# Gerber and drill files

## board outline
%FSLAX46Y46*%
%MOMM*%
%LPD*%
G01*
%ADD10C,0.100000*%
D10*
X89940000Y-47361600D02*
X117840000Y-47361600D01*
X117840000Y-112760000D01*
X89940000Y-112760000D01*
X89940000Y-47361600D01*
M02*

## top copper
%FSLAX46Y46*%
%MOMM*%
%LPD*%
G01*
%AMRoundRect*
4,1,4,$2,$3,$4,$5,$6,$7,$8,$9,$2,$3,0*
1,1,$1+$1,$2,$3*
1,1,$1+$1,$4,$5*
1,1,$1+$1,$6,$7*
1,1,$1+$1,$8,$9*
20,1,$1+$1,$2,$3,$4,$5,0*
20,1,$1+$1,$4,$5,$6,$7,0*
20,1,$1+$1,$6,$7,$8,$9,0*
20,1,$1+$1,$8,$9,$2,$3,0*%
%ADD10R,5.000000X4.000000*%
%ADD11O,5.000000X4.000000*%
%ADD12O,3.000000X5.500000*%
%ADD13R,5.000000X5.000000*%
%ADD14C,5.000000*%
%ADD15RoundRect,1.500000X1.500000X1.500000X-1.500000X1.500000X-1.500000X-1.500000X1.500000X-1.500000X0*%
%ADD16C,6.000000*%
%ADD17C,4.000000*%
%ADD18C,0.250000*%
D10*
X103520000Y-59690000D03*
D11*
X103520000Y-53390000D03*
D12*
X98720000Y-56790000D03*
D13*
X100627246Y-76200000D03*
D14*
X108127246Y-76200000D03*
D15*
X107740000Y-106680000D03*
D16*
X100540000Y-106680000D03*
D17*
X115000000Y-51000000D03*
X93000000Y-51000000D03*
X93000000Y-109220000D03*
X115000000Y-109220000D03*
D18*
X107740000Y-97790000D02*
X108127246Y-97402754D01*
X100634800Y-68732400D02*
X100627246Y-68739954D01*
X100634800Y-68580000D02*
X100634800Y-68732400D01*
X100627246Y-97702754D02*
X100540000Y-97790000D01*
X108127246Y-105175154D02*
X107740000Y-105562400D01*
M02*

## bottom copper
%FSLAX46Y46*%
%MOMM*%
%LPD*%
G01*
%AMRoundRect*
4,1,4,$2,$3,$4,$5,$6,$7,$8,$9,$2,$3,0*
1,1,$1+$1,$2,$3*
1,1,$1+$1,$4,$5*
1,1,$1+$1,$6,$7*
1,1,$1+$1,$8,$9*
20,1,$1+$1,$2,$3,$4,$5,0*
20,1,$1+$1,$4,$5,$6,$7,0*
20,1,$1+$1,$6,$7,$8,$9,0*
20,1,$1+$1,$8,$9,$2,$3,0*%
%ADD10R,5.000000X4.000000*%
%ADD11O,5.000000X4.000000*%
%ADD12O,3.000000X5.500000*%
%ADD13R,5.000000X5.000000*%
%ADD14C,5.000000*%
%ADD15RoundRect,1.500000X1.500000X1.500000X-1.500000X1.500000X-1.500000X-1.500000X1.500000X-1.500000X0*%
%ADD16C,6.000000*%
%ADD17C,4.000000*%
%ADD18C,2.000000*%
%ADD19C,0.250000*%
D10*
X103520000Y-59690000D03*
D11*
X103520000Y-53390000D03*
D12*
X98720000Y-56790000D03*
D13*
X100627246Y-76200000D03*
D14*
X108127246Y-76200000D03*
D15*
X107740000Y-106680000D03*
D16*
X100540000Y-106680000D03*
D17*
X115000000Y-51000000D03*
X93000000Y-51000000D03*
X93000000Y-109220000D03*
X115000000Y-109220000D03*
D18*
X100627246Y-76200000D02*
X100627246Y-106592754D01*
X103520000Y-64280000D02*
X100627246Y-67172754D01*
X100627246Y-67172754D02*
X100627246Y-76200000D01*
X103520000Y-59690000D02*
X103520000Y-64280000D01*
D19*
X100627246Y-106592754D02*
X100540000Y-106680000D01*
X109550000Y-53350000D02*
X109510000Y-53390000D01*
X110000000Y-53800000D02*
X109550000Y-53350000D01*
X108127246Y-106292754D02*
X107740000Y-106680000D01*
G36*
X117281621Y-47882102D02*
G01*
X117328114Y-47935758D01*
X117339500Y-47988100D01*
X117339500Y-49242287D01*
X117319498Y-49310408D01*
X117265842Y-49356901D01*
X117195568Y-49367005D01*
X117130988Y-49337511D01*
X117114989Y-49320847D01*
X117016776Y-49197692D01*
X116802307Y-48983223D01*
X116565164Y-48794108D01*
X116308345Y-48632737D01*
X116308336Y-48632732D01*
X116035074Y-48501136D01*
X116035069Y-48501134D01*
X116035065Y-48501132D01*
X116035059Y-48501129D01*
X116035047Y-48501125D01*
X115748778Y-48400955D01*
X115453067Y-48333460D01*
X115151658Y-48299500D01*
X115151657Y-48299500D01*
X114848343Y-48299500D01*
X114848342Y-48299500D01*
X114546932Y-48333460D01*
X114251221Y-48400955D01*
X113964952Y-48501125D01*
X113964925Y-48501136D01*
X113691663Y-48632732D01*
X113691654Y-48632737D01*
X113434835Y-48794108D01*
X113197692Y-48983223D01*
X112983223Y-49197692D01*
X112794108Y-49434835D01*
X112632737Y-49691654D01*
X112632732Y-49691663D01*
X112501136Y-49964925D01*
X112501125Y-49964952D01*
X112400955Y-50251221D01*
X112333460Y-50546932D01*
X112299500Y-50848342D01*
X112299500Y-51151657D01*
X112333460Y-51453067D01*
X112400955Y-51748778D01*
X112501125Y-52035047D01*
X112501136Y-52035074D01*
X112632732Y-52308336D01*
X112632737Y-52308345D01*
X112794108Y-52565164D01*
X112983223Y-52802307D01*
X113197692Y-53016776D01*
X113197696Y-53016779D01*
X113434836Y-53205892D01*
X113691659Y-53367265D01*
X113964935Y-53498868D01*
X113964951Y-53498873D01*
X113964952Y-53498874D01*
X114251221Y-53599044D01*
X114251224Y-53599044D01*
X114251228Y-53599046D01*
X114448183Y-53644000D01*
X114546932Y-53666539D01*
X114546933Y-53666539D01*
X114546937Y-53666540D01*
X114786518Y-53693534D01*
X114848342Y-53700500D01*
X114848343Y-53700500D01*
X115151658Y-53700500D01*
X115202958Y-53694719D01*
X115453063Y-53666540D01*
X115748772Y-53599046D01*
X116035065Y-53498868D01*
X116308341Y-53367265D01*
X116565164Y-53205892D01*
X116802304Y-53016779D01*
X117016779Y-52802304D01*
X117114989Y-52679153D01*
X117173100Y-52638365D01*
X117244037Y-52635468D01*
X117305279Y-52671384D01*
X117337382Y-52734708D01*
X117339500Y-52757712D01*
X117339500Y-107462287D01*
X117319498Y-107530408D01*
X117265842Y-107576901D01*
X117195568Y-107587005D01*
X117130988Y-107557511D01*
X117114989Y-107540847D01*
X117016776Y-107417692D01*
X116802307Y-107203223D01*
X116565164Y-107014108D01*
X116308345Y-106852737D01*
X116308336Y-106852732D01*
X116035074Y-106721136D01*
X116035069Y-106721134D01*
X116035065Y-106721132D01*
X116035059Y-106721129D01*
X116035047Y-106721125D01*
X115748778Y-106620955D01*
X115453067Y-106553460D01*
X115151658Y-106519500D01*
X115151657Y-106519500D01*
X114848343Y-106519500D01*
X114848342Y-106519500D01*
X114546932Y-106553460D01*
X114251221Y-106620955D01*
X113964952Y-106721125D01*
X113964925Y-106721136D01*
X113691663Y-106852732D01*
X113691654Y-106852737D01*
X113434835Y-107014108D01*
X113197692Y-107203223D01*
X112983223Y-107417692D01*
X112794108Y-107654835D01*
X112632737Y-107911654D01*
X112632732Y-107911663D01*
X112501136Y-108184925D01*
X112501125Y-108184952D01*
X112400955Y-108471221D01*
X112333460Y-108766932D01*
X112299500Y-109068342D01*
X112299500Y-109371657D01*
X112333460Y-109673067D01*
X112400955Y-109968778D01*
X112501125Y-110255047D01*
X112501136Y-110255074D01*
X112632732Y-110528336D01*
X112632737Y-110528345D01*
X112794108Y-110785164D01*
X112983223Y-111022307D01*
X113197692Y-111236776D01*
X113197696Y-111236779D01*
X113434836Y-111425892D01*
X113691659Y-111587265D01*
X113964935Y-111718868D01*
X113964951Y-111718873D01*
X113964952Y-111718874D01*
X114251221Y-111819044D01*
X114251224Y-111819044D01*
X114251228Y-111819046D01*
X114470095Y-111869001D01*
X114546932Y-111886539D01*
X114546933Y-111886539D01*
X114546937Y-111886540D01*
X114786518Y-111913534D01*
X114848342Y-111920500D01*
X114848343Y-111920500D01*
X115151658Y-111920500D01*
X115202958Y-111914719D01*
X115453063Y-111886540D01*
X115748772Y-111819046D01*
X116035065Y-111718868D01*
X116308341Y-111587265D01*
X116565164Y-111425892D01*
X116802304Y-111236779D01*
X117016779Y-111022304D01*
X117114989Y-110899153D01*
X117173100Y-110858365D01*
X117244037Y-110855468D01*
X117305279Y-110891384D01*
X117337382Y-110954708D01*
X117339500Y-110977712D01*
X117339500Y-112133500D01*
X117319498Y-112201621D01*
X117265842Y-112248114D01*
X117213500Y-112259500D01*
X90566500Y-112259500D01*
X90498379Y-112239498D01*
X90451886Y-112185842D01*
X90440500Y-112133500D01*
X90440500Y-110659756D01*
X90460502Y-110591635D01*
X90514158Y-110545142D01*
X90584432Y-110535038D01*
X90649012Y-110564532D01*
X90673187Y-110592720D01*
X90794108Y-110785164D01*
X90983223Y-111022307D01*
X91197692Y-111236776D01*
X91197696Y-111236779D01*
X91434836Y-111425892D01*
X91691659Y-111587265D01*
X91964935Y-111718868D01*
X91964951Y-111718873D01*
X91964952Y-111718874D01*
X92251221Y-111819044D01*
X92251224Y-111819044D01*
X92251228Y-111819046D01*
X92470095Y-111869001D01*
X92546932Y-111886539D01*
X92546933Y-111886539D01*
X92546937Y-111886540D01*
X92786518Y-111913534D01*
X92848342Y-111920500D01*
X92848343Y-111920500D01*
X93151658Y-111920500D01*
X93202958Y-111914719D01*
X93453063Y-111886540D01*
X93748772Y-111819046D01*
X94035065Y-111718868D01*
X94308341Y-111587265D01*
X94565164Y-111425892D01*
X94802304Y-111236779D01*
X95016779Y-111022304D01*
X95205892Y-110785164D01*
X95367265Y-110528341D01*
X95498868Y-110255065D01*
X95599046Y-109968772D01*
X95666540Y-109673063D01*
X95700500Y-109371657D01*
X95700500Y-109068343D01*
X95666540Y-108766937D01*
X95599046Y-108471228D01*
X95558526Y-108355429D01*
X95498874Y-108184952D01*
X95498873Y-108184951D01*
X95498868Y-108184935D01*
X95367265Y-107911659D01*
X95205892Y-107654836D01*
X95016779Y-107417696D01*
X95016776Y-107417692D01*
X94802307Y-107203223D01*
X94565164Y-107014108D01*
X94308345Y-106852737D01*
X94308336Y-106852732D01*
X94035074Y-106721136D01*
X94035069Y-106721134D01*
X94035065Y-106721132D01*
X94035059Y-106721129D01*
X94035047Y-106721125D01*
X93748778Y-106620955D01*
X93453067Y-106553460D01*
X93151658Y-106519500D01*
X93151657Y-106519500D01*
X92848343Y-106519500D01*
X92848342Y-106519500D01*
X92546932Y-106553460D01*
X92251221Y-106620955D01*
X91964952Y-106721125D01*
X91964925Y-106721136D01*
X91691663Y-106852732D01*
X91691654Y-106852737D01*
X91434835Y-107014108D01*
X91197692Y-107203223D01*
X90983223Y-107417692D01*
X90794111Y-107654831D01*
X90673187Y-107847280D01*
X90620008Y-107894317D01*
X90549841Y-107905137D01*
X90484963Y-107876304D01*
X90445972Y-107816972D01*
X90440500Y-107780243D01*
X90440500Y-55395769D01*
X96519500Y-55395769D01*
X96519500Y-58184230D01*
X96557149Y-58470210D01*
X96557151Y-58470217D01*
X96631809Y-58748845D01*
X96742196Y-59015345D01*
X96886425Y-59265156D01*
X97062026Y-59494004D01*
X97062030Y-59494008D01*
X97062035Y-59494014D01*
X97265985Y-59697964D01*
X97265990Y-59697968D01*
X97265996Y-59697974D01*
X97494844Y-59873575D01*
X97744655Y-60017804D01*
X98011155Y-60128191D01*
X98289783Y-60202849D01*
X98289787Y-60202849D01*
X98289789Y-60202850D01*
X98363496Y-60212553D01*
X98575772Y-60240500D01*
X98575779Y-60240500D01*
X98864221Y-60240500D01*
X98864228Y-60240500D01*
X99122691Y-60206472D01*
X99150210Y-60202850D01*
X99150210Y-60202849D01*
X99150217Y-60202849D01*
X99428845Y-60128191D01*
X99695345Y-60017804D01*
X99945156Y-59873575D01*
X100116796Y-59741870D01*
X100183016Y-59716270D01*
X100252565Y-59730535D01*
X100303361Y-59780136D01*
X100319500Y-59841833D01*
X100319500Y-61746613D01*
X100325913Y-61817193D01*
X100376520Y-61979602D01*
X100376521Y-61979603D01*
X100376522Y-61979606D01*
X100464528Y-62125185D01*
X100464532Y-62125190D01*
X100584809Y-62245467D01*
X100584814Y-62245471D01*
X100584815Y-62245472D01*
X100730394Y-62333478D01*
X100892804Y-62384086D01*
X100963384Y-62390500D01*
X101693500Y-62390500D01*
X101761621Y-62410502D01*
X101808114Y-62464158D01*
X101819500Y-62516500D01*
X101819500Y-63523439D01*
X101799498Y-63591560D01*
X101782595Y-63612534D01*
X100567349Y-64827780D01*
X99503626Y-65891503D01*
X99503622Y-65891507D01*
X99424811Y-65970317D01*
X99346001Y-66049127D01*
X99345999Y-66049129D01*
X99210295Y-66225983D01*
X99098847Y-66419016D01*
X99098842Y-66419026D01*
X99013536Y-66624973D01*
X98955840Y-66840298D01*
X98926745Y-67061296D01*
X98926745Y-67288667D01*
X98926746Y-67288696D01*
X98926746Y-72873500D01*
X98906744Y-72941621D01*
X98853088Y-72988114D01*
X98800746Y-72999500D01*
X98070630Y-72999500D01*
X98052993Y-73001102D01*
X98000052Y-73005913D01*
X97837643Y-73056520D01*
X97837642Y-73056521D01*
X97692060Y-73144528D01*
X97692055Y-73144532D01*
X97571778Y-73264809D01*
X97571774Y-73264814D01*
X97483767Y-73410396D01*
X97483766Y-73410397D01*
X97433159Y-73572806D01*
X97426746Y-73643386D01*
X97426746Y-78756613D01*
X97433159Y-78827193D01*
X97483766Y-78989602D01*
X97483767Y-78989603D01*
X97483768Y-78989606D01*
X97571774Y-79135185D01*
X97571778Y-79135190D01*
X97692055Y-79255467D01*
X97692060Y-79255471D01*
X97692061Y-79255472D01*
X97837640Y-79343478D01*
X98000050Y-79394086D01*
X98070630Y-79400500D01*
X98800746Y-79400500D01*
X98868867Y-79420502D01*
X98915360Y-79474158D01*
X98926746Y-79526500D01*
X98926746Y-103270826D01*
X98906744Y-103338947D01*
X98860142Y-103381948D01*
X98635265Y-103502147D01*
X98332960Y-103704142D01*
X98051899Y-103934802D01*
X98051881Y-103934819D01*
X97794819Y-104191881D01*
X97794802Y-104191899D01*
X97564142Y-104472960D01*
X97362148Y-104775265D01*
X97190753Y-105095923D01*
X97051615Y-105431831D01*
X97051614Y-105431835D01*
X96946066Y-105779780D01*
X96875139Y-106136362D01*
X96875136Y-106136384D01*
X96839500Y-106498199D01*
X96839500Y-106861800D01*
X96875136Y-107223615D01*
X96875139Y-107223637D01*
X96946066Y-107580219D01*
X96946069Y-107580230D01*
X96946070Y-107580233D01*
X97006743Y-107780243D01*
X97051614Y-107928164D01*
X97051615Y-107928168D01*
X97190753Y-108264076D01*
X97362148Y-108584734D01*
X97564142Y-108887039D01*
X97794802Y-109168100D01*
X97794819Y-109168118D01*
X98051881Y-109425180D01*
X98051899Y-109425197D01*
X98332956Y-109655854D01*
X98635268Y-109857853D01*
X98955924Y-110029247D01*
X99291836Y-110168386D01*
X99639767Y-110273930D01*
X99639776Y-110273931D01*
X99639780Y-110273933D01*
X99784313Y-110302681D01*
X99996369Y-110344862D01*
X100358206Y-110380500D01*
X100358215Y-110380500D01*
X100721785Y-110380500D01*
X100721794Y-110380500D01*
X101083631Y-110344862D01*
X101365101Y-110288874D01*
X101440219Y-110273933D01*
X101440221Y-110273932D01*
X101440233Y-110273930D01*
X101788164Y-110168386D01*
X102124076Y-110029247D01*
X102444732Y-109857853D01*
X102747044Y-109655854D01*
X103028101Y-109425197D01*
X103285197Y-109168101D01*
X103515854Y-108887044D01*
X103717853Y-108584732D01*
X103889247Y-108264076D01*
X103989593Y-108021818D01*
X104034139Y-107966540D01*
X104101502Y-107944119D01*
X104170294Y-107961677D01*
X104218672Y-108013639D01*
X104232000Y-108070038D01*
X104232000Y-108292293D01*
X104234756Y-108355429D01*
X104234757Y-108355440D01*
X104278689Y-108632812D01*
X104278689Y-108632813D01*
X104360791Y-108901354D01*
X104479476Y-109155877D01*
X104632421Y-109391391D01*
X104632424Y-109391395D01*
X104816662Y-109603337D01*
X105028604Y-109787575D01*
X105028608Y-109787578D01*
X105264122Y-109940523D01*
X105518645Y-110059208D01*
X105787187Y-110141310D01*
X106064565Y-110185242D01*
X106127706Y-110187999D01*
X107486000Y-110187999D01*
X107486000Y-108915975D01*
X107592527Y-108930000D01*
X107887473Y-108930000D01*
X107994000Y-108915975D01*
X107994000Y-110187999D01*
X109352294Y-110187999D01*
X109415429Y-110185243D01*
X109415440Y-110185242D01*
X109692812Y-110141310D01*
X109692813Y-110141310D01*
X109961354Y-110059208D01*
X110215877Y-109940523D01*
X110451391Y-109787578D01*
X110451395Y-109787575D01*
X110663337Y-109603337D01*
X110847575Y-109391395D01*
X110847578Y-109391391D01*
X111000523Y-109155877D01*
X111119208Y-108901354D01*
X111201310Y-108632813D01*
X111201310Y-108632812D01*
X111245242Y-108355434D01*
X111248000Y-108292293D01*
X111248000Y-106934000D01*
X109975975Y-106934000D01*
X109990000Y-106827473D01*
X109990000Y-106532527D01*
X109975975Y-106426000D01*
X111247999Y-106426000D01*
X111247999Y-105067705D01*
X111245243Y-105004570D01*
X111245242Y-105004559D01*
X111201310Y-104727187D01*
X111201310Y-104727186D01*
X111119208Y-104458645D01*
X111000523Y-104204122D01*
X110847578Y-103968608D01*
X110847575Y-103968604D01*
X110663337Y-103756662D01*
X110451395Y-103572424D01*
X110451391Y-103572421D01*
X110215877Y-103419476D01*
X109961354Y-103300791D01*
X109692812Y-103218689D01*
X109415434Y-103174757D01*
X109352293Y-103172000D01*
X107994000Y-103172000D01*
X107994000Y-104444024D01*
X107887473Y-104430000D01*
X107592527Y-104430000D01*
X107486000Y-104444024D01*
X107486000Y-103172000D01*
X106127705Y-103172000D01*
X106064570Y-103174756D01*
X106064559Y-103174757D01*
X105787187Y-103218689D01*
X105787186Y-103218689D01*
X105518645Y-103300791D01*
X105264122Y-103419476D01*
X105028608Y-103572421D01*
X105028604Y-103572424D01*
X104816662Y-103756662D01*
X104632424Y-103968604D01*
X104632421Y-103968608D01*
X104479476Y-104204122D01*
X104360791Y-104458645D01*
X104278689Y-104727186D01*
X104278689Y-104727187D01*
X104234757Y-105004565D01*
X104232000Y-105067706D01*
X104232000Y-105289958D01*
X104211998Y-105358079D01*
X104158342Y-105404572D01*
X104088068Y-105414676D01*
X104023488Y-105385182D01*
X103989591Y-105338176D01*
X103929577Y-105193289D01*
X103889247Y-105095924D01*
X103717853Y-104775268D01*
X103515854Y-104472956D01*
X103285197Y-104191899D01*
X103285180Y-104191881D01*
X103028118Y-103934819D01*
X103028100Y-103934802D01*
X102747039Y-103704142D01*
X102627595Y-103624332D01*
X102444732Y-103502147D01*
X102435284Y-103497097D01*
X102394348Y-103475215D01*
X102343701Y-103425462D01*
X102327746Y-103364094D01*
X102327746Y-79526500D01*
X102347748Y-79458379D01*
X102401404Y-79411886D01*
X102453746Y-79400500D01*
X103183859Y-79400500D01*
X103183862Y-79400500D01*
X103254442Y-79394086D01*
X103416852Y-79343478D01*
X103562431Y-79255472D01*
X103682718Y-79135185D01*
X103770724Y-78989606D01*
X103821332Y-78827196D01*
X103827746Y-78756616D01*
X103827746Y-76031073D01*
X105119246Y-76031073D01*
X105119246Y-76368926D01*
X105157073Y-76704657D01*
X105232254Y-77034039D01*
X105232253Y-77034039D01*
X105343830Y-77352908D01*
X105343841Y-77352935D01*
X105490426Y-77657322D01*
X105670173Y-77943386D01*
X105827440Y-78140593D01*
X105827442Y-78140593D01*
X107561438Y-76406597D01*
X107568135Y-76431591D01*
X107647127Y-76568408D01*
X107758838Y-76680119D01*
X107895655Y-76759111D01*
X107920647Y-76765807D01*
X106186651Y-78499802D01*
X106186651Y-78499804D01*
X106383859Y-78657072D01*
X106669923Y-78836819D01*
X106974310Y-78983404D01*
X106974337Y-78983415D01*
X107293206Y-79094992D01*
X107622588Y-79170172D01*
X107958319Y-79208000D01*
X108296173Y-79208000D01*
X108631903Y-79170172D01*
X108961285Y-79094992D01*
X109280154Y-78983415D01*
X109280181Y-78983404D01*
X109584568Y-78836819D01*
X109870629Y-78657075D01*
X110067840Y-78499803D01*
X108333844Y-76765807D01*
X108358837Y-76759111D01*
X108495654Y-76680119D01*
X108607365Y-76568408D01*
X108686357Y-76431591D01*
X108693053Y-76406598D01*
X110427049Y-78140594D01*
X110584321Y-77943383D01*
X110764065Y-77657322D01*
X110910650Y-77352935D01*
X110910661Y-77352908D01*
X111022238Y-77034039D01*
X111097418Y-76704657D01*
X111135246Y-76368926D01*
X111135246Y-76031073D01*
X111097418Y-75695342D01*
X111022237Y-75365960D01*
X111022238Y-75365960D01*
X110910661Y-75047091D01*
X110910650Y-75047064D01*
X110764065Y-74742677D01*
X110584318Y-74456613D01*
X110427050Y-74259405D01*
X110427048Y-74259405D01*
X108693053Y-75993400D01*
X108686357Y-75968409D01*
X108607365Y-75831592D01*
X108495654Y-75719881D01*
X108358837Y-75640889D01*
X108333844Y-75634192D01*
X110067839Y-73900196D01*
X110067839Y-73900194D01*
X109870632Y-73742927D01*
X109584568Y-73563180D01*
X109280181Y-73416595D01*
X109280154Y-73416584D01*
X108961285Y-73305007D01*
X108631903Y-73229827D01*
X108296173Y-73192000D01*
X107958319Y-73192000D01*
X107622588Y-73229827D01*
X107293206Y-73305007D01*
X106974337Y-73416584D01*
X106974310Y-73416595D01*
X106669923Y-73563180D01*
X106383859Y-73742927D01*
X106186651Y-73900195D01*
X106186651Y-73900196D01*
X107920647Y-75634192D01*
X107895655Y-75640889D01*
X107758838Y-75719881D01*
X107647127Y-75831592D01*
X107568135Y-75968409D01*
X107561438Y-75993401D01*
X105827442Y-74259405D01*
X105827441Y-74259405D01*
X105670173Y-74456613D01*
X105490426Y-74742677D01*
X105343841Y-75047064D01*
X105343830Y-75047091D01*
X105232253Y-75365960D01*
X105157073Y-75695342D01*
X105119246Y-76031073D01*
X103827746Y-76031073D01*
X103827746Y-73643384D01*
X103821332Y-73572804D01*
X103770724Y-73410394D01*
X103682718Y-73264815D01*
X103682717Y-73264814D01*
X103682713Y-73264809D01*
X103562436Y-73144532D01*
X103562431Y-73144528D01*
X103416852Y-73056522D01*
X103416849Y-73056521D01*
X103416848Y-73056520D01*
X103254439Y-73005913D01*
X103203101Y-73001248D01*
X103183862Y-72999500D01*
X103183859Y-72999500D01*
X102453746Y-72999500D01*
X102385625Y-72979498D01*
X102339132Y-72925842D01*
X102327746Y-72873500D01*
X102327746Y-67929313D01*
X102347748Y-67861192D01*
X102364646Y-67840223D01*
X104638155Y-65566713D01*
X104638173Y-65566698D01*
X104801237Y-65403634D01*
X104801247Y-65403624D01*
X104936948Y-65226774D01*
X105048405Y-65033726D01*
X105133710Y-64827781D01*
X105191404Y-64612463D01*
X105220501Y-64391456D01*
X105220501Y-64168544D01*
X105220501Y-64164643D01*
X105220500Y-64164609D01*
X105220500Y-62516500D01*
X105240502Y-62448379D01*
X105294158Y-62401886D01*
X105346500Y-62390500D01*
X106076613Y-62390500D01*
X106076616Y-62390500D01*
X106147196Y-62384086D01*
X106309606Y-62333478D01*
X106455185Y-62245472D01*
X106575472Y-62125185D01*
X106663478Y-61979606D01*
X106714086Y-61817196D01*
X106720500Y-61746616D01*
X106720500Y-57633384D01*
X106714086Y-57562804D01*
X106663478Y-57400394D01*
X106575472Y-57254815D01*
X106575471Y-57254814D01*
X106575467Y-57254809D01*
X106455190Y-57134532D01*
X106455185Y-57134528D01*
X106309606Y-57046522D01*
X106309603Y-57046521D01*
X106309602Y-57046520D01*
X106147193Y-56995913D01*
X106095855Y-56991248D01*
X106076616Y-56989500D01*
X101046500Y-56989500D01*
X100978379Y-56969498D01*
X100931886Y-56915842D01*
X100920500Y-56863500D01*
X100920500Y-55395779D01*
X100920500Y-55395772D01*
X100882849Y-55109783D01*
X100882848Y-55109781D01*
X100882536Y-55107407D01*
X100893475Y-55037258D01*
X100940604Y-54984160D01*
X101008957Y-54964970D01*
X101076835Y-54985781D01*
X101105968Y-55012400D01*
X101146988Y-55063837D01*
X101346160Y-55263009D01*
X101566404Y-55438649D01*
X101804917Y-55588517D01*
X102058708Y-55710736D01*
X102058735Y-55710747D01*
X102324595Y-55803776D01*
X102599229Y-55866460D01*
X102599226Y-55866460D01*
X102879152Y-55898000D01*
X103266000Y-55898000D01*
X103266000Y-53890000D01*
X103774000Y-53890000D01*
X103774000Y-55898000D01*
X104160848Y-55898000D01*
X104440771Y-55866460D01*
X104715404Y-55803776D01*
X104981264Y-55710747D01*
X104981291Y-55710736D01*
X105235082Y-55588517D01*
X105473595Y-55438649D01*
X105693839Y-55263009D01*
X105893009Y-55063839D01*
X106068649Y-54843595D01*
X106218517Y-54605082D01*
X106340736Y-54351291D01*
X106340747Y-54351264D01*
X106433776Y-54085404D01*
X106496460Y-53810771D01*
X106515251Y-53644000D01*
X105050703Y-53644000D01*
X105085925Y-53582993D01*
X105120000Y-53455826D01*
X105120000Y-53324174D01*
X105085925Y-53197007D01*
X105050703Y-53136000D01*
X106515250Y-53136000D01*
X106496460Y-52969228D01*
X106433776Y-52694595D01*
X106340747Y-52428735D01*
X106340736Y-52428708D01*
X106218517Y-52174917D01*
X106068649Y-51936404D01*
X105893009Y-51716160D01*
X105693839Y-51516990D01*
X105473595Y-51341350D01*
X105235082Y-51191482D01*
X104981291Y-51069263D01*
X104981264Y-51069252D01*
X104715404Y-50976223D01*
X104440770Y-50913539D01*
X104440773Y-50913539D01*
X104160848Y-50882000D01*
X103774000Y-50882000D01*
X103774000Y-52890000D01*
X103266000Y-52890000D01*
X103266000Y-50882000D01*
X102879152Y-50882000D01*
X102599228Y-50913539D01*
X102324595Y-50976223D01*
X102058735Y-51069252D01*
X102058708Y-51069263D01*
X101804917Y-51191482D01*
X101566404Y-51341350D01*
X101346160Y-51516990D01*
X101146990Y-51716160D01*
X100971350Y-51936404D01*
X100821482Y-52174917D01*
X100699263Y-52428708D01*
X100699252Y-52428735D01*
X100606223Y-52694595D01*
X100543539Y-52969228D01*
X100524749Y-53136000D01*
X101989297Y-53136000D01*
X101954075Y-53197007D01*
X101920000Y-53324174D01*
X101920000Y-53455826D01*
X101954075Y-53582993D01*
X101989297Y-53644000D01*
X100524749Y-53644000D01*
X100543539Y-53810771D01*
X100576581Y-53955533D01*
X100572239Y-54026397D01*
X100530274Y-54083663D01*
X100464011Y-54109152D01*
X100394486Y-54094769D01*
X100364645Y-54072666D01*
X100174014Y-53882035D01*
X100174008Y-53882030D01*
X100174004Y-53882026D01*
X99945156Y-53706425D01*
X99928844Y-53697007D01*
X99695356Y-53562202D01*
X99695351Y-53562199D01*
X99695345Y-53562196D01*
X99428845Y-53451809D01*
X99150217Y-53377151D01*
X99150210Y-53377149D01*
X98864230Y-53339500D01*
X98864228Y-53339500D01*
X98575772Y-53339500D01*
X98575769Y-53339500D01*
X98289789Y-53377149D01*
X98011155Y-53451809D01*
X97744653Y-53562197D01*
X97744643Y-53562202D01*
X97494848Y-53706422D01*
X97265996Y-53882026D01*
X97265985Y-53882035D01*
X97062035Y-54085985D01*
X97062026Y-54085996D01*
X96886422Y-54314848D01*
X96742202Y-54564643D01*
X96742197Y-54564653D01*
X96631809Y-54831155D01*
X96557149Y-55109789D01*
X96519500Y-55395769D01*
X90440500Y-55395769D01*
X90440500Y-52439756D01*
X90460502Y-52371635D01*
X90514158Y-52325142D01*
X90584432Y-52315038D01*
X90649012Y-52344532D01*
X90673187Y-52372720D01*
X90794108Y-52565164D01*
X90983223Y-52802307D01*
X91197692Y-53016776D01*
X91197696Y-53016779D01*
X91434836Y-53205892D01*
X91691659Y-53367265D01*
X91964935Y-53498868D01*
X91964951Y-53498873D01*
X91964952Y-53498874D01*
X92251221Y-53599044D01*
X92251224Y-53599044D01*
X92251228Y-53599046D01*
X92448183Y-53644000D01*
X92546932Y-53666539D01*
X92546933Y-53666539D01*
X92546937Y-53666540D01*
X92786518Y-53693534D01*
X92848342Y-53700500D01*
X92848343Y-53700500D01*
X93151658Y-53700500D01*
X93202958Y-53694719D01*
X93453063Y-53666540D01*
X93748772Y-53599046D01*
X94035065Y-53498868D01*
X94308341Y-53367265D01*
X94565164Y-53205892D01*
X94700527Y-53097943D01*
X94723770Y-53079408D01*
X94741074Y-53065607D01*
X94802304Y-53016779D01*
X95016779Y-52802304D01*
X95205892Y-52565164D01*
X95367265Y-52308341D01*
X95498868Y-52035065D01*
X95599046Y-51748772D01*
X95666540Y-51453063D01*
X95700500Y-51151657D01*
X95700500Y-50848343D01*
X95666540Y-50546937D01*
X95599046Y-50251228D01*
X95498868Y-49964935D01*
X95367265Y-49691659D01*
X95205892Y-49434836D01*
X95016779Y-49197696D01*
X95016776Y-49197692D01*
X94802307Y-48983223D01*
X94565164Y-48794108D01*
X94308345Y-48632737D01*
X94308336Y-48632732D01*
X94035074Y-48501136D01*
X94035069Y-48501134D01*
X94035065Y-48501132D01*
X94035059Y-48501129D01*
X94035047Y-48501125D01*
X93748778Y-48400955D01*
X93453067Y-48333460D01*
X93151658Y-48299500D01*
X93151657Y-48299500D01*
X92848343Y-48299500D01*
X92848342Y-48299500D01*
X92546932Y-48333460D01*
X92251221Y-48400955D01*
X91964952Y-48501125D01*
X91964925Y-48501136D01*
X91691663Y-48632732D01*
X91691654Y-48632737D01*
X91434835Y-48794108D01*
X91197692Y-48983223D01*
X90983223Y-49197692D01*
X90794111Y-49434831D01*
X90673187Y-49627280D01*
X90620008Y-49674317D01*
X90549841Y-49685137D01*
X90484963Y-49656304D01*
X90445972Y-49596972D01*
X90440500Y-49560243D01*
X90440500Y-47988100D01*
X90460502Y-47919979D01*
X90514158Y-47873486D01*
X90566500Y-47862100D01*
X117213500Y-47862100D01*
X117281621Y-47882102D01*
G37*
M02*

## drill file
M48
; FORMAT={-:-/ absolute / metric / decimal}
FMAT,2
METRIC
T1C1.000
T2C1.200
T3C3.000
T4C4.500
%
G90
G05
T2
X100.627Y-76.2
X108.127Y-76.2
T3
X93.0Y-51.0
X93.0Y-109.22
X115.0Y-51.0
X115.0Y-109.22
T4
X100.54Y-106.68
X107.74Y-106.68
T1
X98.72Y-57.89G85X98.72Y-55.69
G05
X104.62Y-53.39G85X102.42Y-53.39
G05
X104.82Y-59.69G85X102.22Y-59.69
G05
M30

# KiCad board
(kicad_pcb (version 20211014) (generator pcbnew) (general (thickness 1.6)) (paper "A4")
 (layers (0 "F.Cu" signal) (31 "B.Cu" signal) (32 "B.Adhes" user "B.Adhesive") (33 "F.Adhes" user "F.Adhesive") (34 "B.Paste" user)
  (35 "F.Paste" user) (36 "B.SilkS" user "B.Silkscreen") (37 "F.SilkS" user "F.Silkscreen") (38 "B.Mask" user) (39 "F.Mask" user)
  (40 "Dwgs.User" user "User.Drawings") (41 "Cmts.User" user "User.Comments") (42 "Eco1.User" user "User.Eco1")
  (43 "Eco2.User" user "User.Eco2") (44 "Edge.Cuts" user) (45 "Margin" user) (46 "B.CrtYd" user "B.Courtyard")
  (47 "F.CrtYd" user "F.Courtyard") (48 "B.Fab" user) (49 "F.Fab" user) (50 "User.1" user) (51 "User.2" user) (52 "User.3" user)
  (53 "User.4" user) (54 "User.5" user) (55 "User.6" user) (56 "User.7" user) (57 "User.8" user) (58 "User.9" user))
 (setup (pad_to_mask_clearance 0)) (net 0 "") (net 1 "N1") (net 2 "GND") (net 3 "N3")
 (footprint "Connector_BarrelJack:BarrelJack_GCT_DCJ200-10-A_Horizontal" (layer "F.Cu") (at 103.52 59.69 180)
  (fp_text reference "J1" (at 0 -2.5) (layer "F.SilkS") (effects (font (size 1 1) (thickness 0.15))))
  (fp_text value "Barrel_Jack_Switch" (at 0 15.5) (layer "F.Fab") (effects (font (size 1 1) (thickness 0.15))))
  (pad "1" thru_hole rect (at 0 0 180) (size 5 4) (drill oval 3.6 1) (layers *.Cu *.Mask) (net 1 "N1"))
  (pad "2" thru_hole oval (at 0 6.3 180) (size 5 4) (drill oval 3.2 1) (layers *.Cu *.Mask) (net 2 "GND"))
  (pad "3" thru_hole oval (at 4.8 2.9 180) (size 3 5.5) (drill oval 1 3.2) (layers *.Cu *.Mask) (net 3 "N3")))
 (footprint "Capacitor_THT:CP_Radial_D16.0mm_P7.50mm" (layer "F.Cu") (at 100.627246 76.2)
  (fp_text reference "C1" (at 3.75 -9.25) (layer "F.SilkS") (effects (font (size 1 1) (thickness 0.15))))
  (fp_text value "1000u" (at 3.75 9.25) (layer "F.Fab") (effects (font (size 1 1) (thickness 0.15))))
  (pad "1" thru_hole rect (at 0 0) (size 5 5) (drill 1.2) (layers *.Cu *.Mask) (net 1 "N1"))
  (pad "2" thru_hole circle (at 7.5 0) (size 5 5) (drill 1.2) (layers *.Cu *.Mask) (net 2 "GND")))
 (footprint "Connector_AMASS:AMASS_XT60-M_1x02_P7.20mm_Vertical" (layer "F.Cu") (at 107.74 106.68 180)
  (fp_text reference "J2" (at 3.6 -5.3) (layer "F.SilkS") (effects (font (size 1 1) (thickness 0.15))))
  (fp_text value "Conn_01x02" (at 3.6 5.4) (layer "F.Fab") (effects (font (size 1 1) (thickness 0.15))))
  (pad "1" thru_hole roundrect (at 0 0 180) (size 6 6) (drill 4.5) (layers *.Cu *.Mask) (roundrect_rratio 0.25) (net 2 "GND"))
  (pad "2" thru_hole circle (at 7.2 0 180) (size 6 6) (drill 4.5) (layers *.Cu *.Mask) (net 1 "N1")))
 (gr_rect (start 89.94 47.3616) (end 117.84 112.76) (layer "Edge.Cuts") (width 0.1) (fill none))
 (segment (start 107.74 97.79) (end 108.127246 97.402754) (width 0.25) (layer "F.Cu") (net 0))
 (via (at 115 51) (size 4) (drill 3) (layers "F.Cu" "B.Cu") (free) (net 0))
 (via (at 93 51) (size 4) (drill 3) (layers "F.Cu" "B.Cu") (free) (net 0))
 (via (at 93 109.22) (size 4) (drill 3) (layers "F.Cu" "B.Cu") (free) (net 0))
 (via (at 115 109.22) (size 4) (drill 3) (layers "F.Cu" "B.Cu") (free) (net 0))
 (segment (start 100.6348 68.7324) (end 100.627246 68.739954) (width 0.25) (layer "F.Cu") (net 1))
 (segment (start 100.6348 68.58) (end 100.6348 68.7324) (width 0.25) (layer "F.Cu") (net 1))
 (segment (start 100.627246 97.702754) (end 100.54 97.79) (width 0.25) (layer "F.Cu") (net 1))
 (segment (start 100.627246 76.2) (end 100.627246 106.592754) (width 2) (layer "B.Cu") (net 1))
 (segment (start 103.52 64.28) (end 100.627246 67.172754) (width 2) (layer "B.Cu") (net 1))
 (segment (start 100.627246 67.172754) (end 100.627246 76.2) (width 2) (layer "B.Cu") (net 1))
 (segment (start 103.52 59.69) (end 103.52 64.28) (width 2) (layer "B.Cu") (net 1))
 (segment (start 100.627246 106.592754) (end 100.54 106.68) (width 0.25) (layer "B.Cu") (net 1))
 (segment (start 108.127246 105.175154) (end 107.74 105.5624) (width 0.25) (layer "F.Cu") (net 2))
 (segment (start 109.55 53.35) (end 109.51 53.39) (width 0.25) (layer "B.Cu") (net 2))
 (segment (start 110 53.8) (end 109.55 53.35) (width 0.25) (layer "B.Cu") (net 2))
 (segment (start 108.127246 106.292754) (end 107.74 106.68) (width 0.25) (layer "B.Cu") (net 2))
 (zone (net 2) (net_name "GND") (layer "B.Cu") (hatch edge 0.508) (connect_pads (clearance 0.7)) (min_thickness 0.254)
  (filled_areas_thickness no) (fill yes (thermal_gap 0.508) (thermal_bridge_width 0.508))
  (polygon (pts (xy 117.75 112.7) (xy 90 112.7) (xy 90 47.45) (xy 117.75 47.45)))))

